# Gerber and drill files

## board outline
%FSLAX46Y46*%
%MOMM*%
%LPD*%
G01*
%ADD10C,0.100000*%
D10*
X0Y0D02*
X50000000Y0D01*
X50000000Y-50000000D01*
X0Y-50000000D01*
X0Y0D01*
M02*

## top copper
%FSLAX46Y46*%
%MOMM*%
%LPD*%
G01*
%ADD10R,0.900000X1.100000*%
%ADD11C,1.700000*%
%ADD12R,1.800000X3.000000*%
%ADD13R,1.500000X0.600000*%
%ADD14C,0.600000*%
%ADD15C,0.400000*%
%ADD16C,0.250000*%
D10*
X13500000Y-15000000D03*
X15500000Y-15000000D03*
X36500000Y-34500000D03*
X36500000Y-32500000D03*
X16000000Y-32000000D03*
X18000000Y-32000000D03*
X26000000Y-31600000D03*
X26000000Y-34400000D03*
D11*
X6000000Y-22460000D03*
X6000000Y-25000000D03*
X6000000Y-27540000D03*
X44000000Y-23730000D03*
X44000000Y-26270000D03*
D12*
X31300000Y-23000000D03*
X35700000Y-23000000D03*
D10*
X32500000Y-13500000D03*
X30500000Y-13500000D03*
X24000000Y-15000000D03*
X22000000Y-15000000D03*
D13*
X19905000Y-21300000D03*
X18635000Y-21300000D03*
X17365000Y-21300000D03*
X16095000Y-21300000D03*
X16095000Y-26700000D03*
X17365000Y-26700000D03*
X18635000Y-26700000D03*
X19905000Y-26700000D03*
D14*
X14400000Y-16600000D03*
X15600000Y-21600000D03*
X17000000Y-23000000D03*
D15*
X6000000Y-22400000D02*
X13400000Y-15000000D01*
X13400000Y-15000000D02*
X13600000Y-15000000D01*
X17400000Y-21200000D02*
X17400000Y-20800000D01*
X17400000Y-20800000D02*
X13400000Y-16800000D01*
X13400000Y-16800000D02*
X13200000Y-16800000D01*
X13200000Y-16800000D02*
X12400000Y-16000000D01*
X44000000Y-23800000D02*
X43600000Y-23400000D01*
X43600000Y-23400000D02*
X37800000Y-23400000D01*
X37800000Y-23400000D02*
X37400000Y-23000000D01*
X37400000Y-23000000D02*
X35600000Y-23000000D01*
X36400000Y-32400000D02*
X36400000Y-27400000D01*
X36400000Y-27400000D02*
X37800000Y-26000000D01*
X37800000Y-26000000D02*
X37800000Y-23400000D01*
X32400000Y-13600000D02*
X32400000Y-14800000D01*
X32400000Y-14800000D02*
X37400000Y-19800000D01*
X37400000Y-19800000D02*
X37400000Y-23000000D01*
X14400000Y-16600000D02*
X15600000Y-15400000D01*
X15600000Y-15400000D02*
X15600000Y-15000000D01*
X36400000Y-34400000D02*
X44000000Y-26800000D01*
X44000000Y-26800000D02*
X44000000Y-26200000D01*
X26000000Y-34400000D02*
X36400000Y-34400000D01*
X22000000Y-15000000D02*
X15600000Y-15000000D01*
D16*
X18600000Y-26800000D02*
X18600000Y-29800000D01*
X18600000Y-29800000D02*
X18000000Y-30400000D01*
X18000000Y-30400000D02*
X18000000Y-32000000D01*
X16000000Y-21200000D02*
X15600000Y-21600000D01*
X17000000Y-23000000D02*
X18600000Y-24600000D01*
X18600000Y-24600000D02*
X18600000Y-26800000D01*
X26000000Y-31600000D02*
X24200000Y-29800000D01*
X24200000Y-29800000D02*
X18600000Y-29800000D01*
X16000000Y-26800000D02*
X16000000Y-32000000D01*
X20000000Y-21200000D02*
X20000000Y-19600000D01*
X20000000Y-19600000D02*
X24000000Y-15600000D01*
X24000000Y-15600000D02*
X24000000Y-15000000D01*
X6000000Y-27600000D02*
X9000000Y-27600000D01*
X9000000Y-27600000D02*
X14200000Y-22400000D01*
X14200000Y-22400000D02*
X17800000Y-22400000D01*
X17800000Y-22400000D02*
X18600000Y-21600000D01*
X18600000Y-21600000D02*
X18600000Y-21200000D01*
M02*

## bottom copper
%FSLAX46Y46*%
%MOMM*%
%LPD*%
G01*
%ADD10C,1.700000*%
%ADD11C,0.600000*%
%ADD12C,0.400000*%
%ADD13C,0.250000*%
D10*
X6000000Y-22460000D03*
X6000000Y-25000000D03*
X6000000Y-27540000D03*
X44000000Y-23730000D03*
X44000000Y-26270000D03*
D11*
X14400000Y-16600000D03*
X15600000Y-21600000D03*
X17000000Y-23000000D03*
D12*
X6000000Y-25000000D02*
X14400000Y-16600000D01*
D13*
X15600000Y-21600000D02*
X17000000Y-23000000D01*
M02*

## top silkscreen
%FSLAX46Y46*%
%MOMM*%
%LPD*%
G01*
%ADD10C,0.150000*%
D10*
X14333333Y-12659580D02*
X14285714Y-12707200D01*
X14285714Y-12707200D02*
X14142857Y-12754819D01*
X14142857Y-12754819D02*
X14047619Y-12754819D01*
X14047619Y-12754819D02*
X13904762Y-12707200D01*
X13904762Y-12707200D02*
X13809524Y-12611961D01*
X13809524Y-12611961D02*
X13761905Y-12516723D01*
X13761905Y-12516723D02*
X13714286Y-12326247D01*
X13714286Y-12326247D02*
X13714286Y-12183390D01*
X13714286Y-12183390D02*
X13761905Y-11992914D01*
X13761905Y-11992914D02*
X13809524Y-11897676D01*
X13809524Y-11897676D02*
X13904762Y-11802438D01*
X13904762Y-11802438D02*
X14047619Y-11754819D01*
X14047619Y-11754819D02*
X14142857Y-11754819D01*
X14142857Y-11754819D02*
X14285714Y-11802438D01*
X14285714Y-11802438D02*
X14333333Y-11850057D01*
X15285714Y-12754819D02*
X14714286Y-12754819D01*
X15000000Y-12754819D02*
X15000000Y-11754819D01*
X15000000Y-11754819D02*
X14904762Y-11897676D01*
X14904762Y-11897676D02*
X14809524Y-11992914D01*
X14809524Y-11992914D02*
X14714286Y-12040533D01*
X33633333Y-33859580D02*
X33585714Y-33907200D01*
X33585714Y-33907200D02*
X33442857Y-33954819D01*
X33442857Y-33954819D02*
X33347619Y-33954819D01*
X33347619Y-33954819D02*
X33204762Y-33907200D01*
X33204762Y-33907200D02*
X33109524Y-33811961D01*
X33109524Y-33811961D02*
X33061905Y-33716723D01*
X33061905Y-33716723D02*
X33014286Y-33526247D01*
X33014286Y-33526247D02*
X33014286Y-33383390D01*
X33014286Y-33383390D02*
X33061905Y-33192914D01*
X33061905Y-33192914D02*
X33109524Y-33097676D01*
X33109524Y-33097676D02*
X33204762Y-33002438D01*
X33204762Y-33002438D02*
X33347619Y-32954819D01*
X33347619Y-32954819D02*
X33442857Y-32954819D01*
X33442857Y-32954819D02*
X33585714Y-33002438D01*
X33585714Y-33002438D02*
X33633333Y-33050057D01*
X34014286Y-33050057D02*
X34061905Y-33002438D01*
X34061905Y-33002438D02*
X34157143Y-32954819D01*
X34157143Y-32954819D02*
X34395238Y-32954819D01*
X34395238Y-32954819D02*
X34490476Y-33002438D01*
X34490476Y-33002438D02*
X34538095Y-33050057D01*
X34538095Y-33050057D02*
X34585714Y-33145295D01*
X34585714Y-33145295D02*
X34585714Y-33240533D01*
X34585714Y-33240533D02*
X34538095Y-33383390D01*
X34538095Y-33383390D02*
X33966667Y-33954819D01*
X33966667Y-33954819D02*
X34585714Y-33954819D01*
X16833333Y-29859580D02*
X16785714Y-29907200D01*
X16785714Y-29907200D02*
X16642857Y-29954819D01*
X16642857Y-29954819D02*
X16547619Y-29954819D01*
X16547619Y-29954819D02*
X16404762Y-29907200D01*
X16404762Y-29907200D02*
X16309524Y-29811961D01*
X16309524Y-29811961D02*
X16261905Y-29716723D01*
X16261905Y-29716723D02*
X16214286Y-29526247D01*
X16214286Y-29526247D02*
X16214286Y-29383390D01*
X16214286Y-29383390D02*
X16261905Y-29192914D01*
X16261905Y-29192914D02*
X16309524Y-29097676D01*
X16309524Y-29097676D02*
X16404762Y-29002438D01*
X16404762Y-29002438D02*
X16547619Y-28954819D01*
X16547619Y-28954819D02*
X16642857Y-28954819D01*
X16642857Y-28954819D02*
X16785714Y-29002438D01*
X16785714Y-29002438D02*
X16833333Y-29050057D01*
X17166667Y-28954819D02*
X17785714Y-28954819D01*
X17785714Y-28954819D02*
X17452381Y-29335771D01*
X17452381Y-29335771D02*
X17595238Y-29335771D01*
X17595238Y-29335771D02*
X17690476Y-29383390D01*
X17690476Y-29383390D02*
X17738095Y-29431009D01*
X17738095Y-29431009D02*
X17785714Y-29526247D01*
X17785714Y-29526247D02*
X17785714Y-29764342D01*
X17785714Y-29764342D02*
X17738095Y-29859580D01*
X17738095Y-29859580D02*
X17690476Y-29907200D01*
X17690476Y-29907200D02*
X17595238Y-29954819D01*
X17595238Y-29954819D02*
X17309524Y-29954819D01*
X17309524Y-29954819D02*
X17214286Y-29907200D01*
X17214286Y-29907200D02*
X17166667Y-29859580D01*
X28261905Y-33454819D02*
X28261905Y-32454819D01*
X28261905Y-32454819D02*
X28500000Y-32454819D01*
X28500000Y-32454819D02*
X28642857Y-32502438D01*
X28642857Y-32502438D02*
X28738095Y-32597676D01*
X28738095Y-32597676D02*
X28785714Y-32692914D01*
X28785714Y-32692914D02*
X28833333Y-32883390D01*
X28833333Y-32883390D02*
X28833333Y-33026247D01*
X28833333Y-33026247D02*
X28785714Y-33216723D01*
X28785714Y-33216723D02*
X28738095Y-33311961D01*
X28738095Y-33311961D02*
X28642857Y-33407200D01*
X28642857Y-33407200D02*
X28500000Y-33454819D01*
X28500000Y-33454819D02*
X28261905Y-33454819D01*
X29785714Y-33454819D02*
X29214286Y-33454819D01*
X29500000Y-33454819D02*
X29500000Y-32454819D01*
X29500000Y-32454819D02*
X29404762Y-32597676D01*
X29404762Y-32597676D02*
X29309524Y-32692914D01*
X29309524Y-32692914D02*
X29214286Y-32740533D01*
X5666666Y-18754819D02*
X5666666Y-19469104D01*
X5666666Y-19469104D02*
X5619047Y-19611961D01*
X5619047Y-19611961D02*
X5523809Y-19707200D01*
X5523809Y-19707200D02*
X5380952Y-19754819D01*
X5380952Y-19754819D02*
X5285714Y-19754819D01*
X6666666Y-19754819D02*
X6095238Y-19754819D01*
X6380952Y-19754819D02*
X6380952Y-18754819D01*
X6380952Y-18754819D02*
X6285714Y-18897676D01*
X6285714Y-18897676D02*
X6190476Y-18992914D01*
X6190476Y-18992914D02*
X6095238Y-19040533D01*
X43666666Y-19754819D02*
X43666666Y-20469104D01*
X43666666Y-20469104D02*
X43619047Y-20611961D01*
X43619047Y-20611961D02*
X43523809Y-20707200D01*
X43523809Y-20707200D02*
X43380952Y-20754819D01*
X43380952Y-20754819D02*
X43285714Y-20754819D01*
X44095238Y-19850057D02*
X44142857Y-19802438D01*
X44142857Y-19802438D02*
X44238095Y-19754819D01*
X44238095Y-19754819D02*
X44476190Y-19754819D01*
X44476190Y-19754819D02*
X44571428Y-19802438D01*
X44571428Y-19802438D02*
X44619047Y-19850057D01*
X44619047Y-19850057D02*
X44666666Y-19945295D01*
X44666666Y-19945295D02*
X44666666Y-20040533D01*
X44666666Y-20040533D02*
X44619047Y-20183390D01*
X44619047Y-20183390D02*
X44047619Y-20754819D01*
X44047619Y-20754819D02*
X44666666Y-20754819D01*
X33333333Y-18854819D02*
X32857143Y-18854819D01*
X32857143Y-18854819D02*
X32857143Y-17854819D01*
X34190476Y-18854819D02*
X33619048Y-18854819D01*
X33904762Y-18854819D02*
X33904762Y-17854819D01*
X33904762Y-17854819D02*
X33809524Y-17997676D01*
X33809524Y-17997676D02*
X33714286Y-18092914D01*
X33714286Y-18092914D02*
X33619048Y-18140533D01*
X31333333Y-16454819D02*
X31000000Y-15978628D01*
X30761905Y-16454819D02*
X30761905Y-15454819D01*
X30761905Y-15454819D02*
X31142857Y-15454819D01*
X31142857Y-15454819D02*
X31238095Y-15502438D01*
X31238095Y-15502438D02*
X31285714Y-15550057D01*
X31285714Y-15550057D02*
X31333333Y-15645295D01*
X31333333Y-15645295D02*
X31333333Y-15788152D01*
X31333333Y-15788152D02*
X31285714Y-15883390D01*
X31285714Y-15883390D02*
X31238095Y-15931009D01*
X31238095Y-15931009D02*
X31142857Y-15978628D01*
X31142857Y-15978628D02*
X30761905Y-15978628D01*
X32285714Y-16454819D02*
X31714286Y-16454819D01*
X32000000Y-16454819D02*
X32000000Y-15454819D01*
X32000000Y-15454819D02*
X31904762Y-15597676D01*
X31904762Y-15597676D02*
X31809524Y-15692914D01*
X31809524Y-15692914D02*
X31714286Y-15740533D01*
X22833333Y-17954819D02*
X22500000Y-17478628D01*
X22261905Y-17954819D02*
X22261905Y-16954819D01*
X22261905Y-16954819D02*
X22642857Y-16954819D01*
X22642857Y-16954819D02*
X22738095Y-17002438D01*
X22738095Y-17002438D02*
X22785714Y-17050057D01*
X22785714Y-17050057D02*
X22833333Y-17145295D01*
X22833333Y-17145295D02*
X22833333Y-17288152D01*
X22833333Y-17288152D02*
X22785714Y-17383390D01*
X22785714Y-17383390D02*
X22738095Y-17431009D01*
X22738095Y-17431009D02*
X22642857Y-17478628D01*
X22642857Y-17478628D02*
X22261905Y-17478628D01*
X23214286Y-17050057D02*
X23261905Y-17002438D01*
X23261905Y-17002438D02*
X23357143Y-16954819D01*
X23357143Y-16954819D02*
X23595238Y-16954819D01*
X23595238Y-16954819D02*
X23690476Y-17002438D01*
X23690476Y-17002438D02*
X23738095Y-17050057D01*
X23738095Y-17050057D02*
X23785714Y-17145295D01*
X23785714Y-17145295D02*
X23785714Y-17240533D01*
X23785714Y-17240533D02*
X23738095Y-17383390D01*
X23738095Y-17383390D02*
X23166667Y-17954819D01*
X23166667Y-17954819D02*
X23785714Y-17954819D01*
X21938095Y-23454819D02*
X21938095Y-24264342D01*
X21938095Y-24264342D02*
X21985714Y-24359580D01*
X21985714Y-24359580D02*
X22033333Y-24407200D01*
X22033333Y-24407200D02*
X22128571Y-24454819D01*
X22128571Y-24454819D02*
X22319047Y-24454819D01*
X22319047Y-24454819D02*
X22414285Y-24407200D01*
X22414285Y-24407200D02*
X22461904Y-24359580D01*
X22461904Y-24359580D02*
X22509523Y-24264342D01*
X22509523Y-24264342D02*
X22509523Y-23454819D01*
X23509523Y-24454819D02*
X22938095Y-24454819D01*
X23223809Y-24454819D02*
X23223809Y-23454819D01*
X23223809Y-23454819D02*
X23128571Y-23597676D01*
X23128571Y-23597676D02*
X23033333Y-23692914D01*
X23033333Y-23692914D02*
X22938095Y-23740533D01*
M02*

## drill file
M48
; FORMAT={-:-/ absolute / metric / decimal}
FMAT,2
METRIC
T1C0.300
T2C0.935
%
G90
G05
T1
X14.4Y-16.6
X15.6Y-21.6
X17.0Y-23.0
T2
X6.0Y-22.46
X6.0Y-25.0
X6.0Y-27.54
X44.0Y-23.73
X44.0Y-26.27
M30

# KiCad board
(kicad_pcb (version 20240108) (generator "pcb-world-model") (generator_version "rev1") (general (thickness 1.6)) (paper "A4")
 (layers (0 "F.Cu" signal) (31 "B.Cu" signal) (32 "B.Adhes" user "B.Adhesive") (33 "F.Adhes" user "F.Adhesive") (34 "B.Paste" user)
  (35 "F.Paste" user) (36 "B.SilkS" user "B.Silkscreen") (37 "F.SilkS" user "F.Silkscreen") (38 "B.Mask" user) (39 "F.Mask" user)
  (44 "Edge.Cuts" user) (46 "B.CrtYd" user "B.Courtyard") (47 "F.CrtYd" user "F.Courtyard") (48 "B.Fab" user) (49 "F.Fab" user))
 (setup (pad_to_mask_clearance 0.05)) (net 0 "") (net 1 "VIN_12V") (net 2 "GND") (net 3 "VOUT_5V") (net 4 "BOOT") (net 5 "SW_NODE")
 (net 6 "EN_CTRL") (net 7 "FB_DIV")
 (gr_rect (start 0.0 0.0) (end 50.0000 50.0000) (stroke (width 0.1) (type default)) (fill none) (layer "Edge.Cuts"))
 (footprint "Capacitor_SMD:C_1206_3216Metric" (layer "F.Cu") (at 14.5000 15.0000 0)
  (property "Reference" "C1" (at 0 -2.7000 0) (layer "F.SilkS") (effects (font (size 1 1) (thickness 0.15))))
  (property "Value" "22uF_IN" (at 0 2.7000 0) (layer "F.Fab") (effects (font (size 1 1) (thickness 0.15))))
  (pad "1" smd rect (at -1.0000 0.0000) (size 0.9000 1.1000) (layers "F.Cu" "F.Paste" "F.Mask") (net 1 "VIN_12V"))
  (pad "2" smd rect (at 1.0000 0.0000) (size 0.9000 1.1000) (layers "F.Cu" "F.Paste" "F.Mask") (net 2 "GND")))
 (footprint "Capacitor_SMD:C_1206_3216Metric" (layer "F.Cu") (at 36.5000 33.5000 90)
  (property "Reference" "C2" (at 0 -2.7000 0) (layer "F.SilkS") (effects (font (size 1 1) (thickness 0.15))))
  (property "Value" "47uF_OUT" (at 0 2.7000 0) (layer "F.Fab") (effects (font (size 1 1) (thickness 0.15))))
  (pad "1" smd rect (at -1.0000 0.0000) (size 0.9000 1.1000) (layers "F.Cu" "F.Paste" "F.Mask") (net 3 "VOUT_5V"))
  (pad "2" smd rect (at 1.0000 0.0000) (size 0.9000 1.1000) (layers "F.Cu" "F.Paste" "F.Mask") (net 2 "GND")))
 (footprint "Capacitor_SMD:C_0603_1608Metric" (layer "F.Cu") (at 17.0000 32.0000 0)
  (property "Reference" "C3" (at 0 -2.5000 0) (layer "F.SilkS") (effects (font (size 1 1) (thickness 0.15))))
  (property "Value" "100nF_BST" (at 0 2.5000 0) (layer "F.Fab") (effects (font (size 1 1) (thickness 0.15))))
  (pad "1" smd rect (at -1.0000 0.0000) (size 0.9000 1.1000) (layers "F.Cu" "F.Paste" "F.Mask") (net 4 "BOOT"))
  (pad "2" smd rect (at 1.0000 0.0000) (size 0.9000 1.1000) (layers "F.Cu" "F.Paste" "F.Mask") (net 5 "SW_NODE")))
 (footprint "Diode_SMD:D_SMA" (layer "F.Cu") (at 26.0000 33.0000 270)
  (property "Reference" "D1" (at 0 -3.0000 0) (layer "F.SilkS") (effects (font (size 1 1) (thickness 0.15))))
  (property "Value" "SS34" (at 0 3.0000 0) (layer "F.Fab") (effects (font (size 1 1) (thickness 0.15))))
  (pad "1" smd rect (at -1.4000 0.0000) (size 0.9000 1.1000) (layers "F.Cu" "F.Paste" "F.Mask") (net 2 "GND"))
  (pad "2" smd rect (at 1.4000 0.0000) (size 0.9000 1.1000) (layers "F.Cu" "F.Paste" "F.Mask") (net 5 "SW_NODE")))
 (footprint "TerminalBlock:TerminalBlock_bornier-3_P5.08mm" (layer "F.Cu") (at 6.0000 25.0000 0) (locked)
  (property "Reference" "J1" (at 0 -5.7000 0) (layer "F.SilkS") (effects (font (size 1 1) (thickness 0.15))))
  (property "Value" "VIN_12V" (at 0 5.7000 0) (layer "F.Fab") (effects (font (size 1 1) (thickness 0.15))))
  (pad "1" thru_hole circle (at 0.0000 -2.5400) (size 1.7000 1.7000) (drill 0.9350) (layers "*.Cu" "*.Mask") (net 1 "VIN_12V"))
  (pad "2" thru_hole circle (at 0.0000 0.0000) (size 1.7000 1.7000) (drill 0.9350) (layers "*.Cu" "*.Mask") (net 2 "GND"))
  (pad "3" thru_hole circle (at 0.0000 2.5400) (size 1.7000 1.7000) (drill 0.9350) (layers "*.Cu" "*.Mask") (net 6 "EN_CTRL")))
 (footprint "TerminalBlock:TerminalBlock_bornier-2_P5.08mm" (layer "F.Cu") (at 44.0000 25.0000 0) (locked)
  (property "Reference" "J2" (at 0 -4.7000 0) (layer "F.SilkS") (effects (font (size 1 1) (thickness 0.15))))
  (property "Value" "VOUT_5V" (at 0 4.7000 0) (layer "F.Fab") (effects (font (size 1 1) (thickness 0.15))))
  (pad "1" thru_hole circle (at 0.0000 -1.2700) (size 1.7000 1.7000) (drill 0.9350) (layers "*.Cu" "*.Mask") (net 3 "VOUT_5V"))
  (pad "2" thru_hole circle (at 0.0000 1.2700) (size 1.7000 1.7000) (drill 0.9350) (layers "*.Cu" "*.Mask") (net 2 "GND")))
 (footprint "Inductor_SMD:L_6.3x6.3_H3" (layer "F.Cu") (at 33.5000 23.0000 0)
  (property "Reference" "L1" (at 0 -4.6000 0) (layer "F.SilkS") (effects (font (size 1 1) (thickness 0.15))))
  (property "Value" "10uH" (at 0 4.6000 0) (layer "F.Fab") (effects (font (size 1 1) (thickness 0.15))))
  (pad "1" smd rect (at -2.2000 0.0000) (size 1.8000 3.0000) (layers "F.Cu" "F.Paste" "F.Mask") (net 5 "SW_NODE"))
  (pad "2" smd rect (at 2.2000 0.0000) (size 1.8000 3.0000) (layers "F.Cu" "F.Paste" "F.Mask") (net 3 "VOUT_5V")))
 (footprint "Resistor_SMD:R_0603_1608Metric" (layer "F.Cu") (at 31.5000 13.5000 180)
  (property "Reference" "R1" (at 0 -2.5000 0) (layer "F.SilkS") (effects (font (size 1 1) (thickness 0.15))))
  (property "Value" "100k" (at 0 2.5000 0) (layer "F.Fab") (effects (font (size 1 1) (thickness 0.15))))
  (pad "1" smd rect (at -1.0000 0.0000) (size 0.9000 1.1000) (layers "F.Cu" "F.Paste" "F.Mask") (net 3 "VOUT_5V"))
  (pad "2" smd rect (at 1.0000 0.0000) (size 0.9000 1.1000) (layers "F.Cu" "F.Paste" "F.Mask") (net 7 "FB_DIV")))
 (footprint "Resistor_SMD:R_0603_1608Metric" (layer "F.Cu") (at 23.0000 15.0000 180)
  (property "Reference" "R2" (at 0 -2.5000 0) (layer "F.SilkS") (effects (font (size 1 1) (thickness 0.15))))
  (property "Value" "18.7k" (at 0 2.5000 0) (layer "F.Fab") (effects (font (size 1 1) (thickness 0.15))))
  (pad "1" smd rect (at -1.0000 0.0000) (size 0.9000 1.1000) (layers "F.Cu" "F.Paste" "F.Mask") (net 7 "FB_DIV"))
  (pad "2" smd rect (at 1.0000 0.0000) (size 0.9000 1.1000) (layers "F.Cu" "F.Paste" "F.Mask") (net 2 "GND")))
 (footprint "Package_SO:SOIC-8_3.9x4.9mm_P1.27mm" (layer "F.Cu") (at 18.0000 24.0000 270)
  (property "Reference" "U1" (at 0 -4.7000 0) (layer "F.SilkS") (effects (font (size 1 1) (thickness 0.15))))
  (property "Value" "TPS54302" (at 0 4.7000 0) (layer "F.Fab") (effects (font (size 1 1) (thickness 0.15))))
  (pad "1" smd rect (at -2.7000 -1.9050) (size 1.5000 0.6000) (layers "F.Cu" "F.Paste" "F.Mask") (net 4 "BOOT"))
  (pad "2" smd rect (at -2.7000 -0.6350) (size 1.5000 0.6000) (layers "F.Cu" "F.Paste" "F.Mask") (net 1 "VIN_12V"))
  (pad "3" smd rect (at -2.7000 0.6350) (size 1.5000 0.6000) (layers "F.Cu" "F.Paste" "F.Mask") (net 5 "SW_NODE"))
  (pad "4" smd rect (at -2.7000 1.9050) (size 1.5000 0.6000) (layers "F.Cu" "F.Paste" "F.Mask") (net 2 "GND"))
  (pad "5" smd rect (at 2.7000 1.9050) (size 1.5000 0.6000) (layers "F.Cu" "F.Paste" "F.Mask") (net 7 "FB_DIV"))
  (pad "6" smd rect (at 2.7000 0.6350) (size 1.5000 0.6000) (layers "F.Cu" "F.Paste" "F.Mask") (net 6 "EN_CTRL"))
  (pad "7" smd rect (at 2.7000 -0.6350) (size 1.5000 0.6000) (layers "F.Cu" "F.Paste" "F.Mask") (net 1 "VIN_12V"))
  (pad "8" smd rect (at 2.7000 -1.9050) (size 1.5000 0.6000) (layers "F.Cu" "F.Paste" "F.Mask") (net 5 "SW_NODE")))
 (segment (start 6.0000 22.4000) (end 13.4000 15.0000) (width 0.4000) (layer "F.Cu") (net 1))
 (segment (start 13.4000 15.0000) (end 13.6000 15.0000) (width 0.4000) (layer "F.Cu") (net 1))
 (segment (start 17.4000 21.2000) (end 17.4000 20.8000) (width 0.4000) (layer "F.Cu") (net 1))
 (segment (start 17.4000 20.8000) (end 13.4000 16.8000) (width 0.4000) (layer "F.Cu") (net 1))
 (segment (start 13.4000 16.8000) (end 13.2000 16.8000) (width 0.4000) (layer "F.Cu") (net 1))
 (segment (start 13.2000 16.8000) (end 12.4000 16.0000) (width 0.4000) (layer "F.Cu") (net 1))
 (segment (start 44.0000 23.8000) (end 43.6000 23.4000) (width 0.4000) (layer "F.Cu") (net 3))
 (segment (start 43.6000 23.4000) (end 37.8000 23.4000) (width 0.4000) (layer "F.Cu") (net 3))
 (segment (start 37.8000 23.4000) (end 37.4000 23.0000) (width 0.4000) (layer "F.Cu") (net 3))
 (segment (start 37.4000 23.0000) (end 35.6000 23.0000) (width 0.4000) (layer "F.Cu") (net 3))
 (segment (start 36.4000 32.4000) (end 36.4000 27.4000) (width 0.4000) (layer "F.Cu") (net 3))
 (segment (start 36.4000 27.4000) (end 37.8000 26.0000) (width 0.4000) (layer "F.Cu") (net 3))
 (segment (start 37.8000 26.0000) (end 37.8000 23.4000) (width 0.4000) (layer "F.Cu") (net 3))
 (segment (start 32.4000 13.6000) (end 32.4000 14.8000) (width 0.4000) (layer "F.Cu") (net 3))
 (segment (start 32.4000 14.8000) (end 37.4000 19.8000) (width 0.4000) (layer "F.Cu") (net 3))
 (segment (start 37.4000 19.8000) (end 37.4000 23.0000) (width 0.4000) (layer "F.Cu") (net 3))
 (segment (start 6.0000 25.0000) (end 14.4000 16.6000) (width 0.4000) (layer "B.Cu") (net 2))
 (segment (start 14.4000 16.6000) (end 15.6000 15.4000) (width 0.4000) (layer "F.Cu") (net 2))
 (segment (start 15.6000 15.4000) (end 15.6000 15.0000) (width 0.4000) (layer "F.Cu") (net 2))
 (segment (start 36.4000 34.4000) (end 44.0000 26.8000) (width 0.4000) (layer "F.Cu") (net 2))
 (segment (start 44.0000 26.8000) (end 44.0000 26.2000) (width 0.4000) (layer "F.Cu") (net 2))
 (segment (start 26.0000 34.4000) (end 36.4000 34.4000) (width 0.4000) (layer "F.Cu") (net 2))
 (segment (start 22.0000 15.0000) (end 15.6000 15.0000) (width 0.4000) (layer "F.Cu") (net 2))
 (segment (start 18.6000 26.8000) (end 18.6000 29.8000) (width 0.2500) (layer "F.Cu") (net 5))
 (segment (start 18.6000 29.8000) (end 18.0000 30.4000) (width 0.2500) (layer "F.Cu") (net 5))
 (segment (start 18.0000 30.4000) (end 18.0000 32.0000) (width 0.2500) (layer "F.Cu") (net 5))
 (segment (start 16.0000 21.2000) (end 15.6000 21.6000) (width 0.2500) (layer "F.Cu") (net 5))
 (segment (start 15.6000 21.6000) (end 17.0000 23.0000) (width 0.2500) (layer "B.Cu") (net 5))
 (segment (start 17.0000 23.0000) (end 18.6000 24.6000) (width 0.2500) (layer "F.Cu") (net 5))
 (segment (start 18.6000 24.6000) (end 18.6000 26.8000) (width 0.2500) (layer "F.Cu") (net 5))
 (segment (start 26.0000 31.6000) (end 24.2000 29.8000) (width 0.2500) (layer "F.Cu") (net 5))
 (segment (start 24.2000 29.8000) (end 18.6000 29.8000) (width 0.2500) (layer "F.Cu") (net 5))
 (segment (start 16.0000 26.8000) (end 16.0000 32.0000) (width 0.2500) (layer "F.Cu") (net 4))
 (segment (start 20.0000 21.2000) (end 20.0000 19.6000) (width 0.2500) (layer "F.Cu") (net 7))
 (segment (start 20.0000 19.6000) (end 24.0000 15.6000) (width 0.2500) (layer "F.Cu") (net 7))
 (segment (start 24.0000 15.6000) (end 24.0000 15.0000) (width 0.2500) (layer "F.Cu") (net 7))
 (segment (start 6.0000 27.6000) (end 9.0000 27.6000) (width 0.2500) (layer "F.Cu") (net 6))
 (segment (start 9.0000 27.6000) (end 14.2000 22.4000) (width 0.2500) (layer "F.Cu") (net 6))
 (segment (start 14.2000 22.4000) (end 17.8000 22.4000) (width 0.2500) (layer "F.Cu") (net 6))
 (segment (start 17.8000 22.4000) (end 18.6000 21.6000) (width 0.2500) (layer "F.Cu") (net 6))
 (segment (start 18.6000 21.6000) (end 18.6000 21.2000) (width 0.2500) (layer "F.Cu") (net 6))
 (via (at 14.4000 16.6000) (size 0.6000) (drill 0.3000) (layers "F.Cu" "B.Cu") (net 2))
 (via (at 15.6000 21.6000) (size 0.6000) (drill 0.3000) (layers "F.Cu" "B.Cu") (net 5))
 (via (at 17.0000 23.0000) (size 0.6000) (drill 0.3000) (layers "F.Cu" "B.Cu") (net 5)))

